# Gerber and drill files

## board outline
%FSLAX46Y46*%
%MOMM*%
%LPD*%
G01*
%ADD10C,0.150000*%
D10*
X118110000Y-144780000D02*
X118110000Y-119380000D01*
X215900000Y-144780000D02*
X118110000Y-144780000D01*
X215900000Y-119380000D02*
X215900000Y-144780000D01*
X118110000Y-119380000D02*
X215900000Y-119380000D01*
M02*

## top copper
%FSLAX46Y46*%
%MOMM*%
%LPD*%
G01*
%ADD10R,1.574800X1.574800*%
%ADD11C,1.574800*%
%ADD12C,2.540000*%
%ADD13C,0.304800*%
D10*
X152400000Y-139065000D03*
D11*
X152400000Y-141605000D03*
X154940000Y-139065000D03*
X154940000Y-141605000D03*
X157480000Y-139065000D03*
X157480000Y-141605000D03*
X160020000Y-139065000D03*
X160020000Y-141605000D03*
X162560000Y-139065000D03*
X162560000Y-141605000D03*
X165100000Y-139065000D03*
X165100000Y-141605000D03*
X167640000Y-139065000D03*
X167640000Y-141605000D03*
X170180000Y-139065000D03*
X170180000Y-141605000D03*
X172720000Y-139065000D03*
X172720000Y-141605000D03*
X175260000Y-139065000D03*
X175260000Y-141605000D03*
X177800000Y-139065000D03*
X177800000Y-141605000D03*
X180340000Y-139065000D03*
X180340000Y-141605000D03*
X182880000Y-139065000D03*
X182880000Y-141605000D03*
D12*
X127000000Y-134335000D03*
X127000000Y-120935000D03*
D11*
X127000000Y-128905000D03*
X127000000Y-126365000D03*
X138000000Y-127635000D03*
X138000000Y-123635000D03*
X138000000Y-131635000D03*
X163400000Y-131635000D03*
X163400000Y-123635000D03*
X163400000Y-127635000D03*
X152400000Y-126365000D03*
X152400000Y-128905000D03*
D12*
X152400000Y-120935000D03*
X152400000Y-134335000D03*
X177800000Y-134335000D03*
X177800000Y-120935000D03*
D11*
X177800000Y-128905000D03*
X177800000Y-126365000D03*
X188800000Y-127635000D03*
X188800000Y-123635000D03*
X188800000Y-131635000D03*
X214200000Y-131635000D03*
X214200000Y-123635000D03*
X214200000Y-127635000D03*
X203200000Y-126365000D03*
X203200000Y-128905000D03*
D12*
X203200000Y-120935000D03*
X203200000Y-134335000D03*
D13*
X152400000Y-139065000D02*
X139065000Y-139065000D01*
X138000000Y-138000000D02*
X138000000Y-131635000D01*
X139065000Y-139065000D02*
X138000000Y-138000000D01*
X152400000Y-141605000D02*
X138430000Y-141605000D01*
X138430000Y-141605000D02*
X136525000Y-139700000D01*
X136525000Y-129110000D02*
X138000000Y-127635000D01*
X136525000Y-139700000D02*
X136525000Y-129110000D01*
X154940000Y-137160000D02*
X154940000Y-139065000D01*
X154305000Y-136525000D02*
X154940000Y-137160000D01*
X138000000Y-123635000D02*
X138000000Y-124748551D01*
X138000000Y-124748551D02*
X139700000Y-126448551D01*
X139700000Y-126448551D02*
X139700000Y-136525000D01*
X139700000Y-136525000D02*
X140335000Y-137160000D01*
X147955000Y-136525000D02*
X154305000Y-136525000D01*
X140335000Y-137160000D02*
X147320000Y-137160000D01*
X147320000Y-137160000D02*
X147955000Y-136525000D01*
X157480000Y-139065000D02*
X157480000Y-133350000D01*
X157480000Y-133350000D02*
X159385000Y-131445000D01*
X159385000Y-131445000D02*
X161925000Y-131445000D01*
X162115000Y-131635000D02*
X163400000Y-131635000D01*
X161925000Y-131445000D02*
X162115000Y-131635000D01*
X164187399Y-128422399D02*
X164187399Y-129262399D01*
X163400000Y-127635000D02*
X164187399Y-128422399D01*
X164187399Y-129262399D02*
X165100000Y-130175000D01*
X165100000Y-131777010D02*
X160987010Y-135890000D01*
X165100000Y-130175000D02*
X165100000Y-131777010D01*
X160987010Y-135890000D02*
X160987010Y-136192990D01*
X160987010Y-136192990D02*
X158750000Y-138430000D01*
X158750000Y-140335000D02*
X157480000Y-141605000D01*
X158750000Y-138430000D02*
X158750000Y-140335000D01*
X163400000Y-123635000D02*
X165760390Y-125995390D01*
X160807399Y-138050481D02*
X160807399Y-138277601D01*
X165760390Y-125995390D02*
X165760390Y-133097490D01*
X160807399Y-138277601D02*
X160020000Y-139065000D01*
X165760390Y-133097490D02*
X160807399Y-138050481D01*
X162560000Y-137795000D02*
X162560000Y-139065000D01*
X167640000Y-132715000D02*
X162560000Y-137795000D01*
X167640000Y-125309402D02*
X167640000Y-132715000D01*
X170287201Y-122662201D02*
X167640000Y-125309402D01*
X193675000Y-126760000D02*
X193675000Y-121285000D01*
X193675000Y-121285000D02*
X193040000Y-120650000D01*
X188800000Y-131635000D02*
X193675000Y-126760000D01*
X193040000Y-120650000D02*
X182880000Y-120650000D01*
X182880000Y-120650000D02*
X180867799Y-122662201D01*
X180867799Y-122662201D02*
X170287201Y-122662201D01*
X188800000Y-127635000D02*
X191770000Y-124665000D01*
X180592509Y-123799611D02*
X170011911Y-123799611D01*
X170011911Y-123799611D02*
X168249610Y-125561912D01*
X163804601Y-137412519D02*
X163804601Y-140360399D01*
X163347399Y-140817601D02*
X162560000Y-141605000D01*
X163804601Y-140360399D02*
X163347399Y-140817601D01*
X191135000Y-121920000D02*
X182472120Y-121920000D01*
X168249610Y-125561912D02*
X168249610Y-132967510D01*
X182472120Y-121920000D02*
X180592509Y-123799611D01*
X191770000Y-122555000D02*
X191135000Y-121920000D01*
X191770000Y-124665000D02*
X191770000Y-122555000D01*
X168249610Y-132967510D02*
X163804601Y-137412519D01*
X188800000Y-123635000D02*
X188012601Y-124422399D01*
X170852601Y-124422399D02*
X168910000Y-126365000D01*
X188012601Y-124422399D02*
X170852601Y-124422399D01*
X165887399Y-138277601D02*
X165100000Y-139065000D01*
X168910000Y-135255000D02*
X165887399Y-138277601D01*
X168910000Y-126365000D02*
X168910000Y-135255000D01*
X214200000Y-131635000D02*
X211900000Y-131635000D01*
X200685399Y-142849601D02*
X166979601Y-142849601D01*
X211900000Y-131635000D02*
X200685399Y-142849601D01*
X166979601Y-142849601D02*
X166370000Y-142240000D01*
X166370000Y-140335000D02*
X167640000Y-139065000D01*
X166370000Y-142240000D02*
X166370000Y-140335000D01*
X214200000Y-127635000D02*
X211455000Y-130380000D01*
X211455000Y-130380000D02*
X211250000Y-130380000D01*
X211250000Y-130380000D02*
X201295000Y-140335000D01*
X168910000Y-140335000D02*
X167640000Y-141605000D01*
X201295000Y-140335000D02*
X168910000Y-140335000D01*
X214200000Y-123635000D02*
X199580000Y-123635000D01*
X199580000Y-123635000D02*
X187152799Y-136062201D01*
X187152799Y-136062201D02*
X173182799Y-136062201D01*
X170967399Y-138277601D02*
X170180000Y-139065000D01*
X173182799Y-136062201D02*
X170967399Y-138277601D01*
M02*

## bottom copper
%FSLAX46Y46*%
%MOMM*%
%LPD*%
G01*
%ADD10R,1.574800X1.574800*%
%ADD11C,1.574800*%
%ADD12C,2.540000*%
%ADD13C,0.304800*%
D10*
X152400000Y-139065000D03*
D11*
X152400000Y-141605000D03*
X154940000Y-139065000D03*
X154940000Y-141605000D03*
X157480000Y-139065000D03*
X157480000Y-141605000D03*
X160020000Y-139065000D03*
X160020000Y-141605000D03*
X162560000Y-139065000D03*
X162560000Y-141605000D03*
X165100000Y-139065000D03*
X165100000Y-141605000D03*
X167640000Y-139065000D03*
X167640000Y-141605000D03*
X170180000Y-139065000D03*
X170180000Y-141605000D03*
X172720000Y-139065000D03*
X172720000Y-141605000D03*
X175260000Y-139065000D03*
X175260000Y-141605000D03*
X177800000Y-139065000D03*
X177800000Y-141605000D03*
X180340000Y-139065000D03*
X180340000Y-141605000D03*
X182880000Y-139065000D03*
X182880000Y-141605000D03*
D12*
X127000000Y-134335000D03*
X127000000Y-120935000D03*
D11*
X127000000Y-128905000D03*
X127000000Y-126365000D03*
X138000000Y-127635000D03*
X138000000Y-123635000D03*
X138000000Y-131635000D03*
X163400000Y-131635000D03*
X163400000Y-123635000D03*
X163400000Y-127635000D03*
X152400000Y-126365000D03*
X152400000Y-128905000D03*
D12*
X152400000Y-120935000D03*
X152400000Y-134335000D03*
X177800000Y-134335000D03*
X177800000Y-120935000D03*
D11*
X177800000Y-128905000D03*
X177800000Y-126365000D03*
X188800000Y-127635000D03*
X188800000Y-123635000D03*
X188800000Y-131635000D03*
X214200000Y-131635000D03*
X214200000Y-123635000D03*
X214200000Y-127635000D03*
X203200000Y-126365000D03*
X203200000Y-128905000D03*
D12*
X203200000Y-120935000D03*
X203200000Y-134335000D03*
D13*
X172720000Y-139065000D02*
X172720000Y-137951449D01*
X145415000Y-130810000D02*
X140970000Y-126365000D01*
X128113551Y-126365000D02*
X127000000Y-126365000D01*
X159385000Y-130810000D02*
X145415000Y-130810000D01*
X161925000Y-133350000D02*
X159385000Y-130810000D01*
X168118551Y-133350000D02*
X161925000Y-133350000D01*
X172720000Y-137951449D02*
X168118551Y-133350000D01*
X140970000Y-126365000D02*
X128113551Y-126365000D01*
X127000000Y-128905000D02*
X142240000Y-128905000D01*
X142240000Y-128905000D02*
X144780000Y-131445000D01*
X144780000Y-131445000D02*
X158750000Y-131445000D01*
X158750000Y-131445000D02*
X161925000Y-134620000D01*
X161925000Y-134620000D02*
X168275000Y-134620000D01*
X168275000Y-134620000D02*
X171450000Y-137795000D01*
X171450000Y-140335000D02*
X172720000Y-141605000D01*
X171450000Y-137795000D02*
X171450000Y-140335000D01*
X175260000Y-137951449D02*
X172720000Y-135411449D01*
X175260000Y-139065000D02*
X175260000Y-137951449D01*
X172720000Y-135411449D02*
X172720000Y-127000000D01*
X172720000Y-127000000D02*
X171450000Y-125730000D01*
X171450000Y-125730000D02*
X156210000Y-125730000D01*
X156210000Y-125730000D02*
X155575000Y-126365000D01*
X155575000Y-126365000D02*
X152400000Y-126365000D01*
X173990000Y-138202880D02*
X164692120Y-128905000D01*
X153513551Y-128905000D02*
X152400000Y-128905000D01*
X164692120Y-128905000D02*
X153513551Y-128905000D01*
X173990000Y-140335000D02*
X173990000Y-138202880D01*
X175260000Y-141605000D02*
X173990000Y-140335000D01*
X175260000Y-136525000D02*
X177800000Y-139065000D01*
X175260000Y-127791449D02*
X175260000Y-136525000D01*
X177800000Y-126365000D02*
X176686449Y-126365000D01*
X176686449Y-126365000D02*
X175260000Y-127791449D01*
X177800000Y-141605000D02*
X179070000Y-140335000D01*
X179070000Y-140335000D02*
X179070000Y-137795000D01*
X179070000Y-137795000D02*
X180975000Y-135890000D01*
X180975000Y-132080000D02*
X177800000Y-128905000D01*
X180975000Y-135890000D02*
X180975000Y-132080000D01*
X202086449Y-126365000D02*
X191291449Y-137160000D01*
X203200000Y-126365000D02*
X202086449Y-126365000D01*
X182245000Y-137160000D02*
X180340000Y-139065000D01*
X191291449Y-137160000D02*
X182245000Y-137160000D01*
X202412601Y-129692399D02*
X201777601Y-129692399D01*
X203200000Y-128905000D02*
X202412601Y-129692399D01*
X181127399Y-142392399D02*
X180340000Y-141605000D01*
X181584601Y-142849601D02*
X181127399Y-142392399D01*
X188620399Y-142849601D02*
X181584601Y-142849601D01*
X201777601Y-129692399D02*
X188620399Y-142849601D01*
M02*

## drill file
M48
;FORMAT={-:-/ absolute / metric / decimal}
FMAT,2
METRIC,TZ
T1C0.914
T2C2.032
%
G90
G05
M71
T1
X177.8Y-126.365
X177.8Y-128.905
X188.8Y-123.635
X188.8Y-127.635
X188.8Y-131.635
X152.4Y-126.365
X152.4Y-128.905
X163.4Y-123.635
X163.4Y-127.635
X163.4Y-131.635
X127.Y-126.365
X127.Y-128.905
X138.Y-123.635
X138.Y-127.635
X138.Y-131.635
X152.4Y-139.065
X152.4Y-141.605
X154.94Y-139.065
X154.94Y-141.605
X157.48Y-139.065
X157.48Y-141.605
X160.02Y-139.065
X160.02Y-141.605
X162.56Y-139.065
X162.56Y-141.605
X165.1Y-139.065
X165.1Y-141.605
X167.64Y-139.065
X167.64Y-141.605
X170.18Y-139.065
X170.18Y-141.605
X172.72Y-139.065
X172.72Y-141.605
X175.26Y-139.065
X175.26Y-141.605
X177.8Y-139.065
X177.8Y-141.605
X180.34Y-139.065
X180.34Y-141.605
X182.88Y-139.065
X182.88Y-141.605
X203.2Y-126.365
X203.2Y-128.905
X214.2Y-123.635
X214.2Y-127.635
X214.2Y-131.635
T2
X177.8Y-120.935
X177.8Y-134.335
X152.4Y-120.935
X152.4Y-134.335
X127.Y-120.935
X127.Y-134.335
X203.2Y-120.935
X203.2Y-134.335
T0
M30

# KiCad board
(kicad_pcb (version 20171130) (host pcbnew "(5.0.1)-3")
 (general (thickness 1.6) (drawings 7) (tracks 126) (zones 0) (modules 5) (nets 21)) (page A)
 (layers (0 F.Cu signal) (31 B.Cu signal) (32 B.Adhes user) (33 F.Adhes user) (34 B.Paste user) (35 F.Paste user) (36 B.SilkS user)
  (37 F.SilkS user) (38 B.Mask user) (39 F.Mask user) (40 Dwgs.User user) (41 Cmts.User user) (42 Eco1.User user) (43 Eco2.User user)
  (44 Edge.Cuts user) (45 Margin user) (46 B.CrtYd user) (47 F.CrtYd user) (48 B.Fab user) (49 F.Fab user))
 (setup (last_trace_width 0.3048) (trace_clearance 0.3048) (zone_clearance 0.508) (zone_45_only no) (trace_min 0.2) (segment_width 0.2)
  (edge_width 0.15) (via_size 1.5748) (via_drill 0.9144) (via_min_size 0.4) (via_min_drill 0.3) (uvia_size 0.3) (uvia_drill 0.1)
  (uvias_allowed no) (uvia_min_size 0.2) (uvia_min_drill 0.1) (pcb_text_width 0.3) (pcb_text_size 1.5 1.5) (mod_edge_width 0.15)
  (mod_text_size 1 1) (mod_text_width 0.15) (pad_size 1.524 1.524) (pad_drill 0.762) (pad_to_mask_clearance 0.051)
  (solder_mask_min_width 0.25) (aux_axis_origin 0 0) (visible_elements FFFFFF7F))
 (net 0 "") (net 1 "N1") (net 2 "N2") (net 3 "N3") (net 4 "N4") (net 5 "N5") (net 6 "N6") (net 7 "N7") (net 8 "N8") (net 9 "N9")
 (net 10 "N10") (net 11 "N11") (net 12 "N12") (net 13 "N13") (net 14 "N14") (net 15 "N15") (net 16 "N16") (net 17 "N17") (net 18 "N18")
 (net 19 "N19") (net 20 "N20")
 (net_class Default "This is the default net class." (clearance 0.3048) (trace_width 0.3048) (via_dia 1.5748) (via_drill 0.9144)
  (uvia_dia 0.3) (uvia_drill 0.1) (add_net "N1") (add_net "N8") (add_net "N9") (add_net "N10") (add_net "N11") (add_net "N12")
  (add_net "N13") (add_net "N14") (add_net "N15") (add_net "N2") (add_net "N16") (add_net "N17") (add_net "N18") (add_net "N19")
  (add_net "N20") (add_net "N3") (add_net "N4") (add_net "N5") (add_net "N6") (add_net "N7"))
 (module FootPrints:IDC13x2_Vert (layer B.Cu) (at 166.37 140.335)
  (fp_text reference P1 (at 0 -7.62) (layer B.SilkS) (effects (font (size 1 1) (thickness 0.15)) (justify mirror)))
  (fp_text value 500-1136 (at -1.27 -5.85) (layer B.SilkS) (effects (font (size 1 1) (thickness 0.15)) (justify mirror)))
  (pad 1 thru_hole rect (at -13.97 -1.27) (size 1.5748 1.5748) (drill 0.9144) (layers *.Cu *.Mask) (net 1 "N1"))
  (pad 2 thru_hole circle (at -13.97 1.27) (size 1.5748 1.5748) (drill 0.9144) (layers *.Cu *.Mask) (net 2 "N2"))
  (pad 3 thru_hole circle (at -11.43 -1.27) (size 1.5748 1.5748) (drill 0.9144) (layers *.Cu *.Mask) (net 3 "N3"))
  (pad 4 thru_hole circle (at -11.43 1.27) (size 1.5748 1.5748) (drill 0.9144) (layers *.Cu *.Mask))
  (pad 5 thru_hole circle (at -8.89 -1.27) (size 1.5748 1.5748) (drill 0.9144) (layers *.Cu *.Mask) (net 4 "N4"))
  (pad 6 thru_hole circle (at -8.89 1.27) (size 1.5748 1.5748) (drill 0.9144) (layers *.Cu *.Mask) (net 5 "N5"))
  (pad 7 thru_hole circle (at -6.35 -1.27) (size 1.5748 1.5748) (drill 0.9144) (layers *.Cu *.Mask) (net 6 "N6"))
  (pad 8 thru_hole circle (at -6.35 1.27) (size 1.5748 1.5748) (drill 0.9144) (layers *.Cu *.Mask))
  (pad 9 thru_hole circle (at -3.81 -1.27) (size 1.5748 1.5748) (drill 0.9144) (layers *.Cu *.Mask) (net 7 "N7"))
  (pad 10 thru_hole circle (at -3.81 1.27) (size 1.5748 1.5748) (drill 0.9144) (layers *.Cu *.Mask) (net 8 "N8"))
  (pad 11 thru_hole circle (at -1.27 -1.27) (size 1.5748 1.5748) (drill 0.9144) (layers *.Cu *.Mask) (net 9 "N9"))
  (pad 12 thru_hole circle (at -1.27 1.27) (size 1.5748 1.5748) (drill 0.9144) (layers *.Cu *.Mask))
  (pad 13 thru_hole circle (at 1.27 -1.27) (size 1.5748 1.5748) (drill 0.9144) (layers *.Cu *.Mask) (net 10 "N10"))
  (pad 14 thru_hole circle (at 1.27 1.27) (size 1.5748 1.5748) (drill 0.9144) (layers *.Cu *.Mask) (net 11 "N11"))
  (pad 15 thru_hole circle (at 3.81 -1.27) (size 1.5748 1.5748) (drill 0.9144) (layers *.Cu *.Mask) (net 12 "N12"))
  (pad 16 thru_hole circle (at 3.81 1.27) (size 1.5748 1.5748) (drill 0.9144) (layers *.Cu *.Mask))
  (pad 17 thru_hole circle (at 6.35 -1.27) (size 1.5748 1.5748) (drill 0.9144) (layers *.Cu *.Mask) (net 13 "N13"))
  (pad 18 thru_hole circle (at 6.35 1.27) (size 1.5748 1.5748) (drill 0.9144) (layers *.Cu *.Mask) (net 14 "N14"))
  (pad 19 thru_hole circle (at 8.89 -1.27) (size 1.5748 1.5748) (drill 0.9144) (layers *.Cu *.Mask) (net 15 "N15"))
  (pad 20 thru_hole circle (at 8.89 1.27) (size 1.5748 1.5748) (drill 0.9144) (layers *.Cu *.Mask) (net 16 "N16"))
  (pad 21 thru_hole circle (at 11.43 -1.27) (size 1.5748 1.5748) (drill 0.9144) (layers *.Cu *.Mask) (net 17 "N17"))
  (pad 22 thru_hole circle (at 11.43 1.27) (size 1.5748 1.5748) (drill 0.9144) (layers *.Cu *.Mask) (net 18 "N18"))
  (pad 23 thru_hole circle (at 13.97 -1.27) (size 1.5748 1.5748) (drill 0.9144) (layers *.Cu *.Mask) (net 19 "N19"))
  (pad 24 thru_hole circle (at 13.97 1.27) (size 1.5748 1.5748) (drill 0.9144) (layers *.Cu *.Mask) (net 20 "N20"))
  (pad 25 thru_hole circle (at 16.51 -1.27) (size 1.5748 1.5748) (drill 0.9144) (layers *.Cu *.Mask))
  (pad 26 thru_hole circle (at 16.51 1.27) (size 1.5748 1.5748) (drill 0.9144) (layers *.Cu *.Mask)))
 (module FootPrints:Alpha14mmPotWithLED (layer F.Cu) (at 127 127.635 90)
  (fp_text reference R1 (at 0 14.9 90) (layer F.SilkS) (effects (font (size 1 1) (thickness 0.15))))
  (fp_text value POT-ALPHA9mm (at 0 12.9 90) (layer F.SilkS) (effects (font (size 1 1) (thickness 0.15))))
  (pad "" thru_hole circle (at -6.7 0 90) (size 2.54 2.54) (drill 2.032) (layers *.Cu *.Mask F.SilkS))
  (pad "" thru_hole circle (at 6.7 0 90) (size 2.54 2.54) (drill 2.032) (layers *.Cu *.Mask F.SilkS))
  (pad 4 thru_hole circle (at -1.27 0 90) (size 1.5748 1.5748) (drill 0.9144) (layers *.Cu *.Mask F.SilkS) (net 14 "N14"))
  (pad 5 thru_hole circle (at 1.27 0 90) (size 1.5748 1.5748) (drill 0.9144) (layers *.Cu *.Mask F.SilkS) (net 13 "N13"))
  (pad 2 thru_hole circle (at 0 11 90) (size 1.5748 1.5748) (drill 0.9144) (layers *.Cu *.Mask F.SilkS) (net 2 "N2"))
  (pad 3 thru_hole circle (at 4 11 90) (size 1.5748 1.5748) (drill 0.9144) (layers *.Cu *.Mask F.SilkS) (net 3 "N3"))
  (pad 1 thru_hole circle (at -4 11 90) (size 1.5748 1.5748) (drill 0.9144) (layers *.Cu *.Mask F.SilkS) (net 1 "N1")))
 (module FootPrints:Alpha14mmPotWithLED (layer F.Cu) (at 152.4 127.635 90)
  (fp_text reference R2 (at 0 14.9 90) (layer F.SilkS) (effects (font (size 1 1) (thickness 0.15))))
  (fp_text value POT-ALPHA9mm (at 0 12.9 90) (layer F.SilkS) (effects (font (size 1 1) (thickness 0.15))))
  (pad 1 thru_hole circle (at -4 11 90) (size 1.5748 1.5748) (drill 0.9144) (layers *.Cu *.Mask F.SilkS) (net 4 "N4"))
  (pad 3 thru_hole circle (at 4 11 90) (size 1.5748 1.5748) (drill 0.9144) (layers *.Cu *.Mask F.SilkS) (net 6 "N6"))
  (pad 2 thru_hole circle (at 0 11 90) (size 1.5748 1.5748) (drill 0.9144) (layers *.Cu *.Mask F.SilkS) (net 5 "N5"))
  (pad 5 thru_hole circle (at 1.27 0 90) (size 1.5748 1.5748) (drill 0.9144) (layers *.Cu *.Mask F.SilkS) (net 15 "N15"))
  (pad 4 thru_hole circle (at -1.27 0 90) (size 1.5748 1.5748) (drill 0.9144) (layers *.Cu *.Mask F.SilkS) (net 16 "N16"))
  (pad "" thru_hole circle (at 6.7 0 90) (size 2.54 2.54) (drill 2.032) (layers *.Cu *.Mask F.SilkS))
  (pad "" thru_hole circle (at -6.7 0 90) (size 2.54 2.54) (drill 2.032) (layers *.Cu *.Mask F.SilkS)))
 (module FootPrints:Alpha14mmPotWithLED (layer F.Cu) (at 177.8 127.635 90)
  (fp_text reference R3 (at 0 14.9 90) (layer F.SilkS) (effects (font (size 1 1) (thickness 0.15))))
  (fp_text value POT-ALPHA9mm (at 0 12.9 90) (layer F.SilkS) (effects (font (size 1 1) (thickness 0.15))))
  (pad "" thru_hole circle (at -6.7 0 90) (size 2.54 2.54) (drill 2.032) (layers *.Cu *.Mask F.SilkS))
  (pad "" thru_hole circle (at 6.7 0 90) (size 2.54 2.54) (drill 2.032) (layers *.Cu *.Mask F.SilkS))
  (pad 4 thru_hole circle (at -1.27 0 90) (size 1.5748 1.5748) (drill 0.9144) (layers *.Cu *.Mask F.SilkS) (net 18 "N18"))
  (pad 5 thru_hole circle (at 1.27 0 90) (size 1.5748 1.5748) (drill 0.9144) (layers *.Cu *.Mask F.SilkS) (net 17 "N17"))
  (pad 2 thru_hole circle (at 0 11 90) (size 1.5748 1.5748) (drill 0.9144) (layers *.Cu *.Mask F.SilkS) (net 8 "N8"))
  (pad 3 thru_hole circle (at 4 11 90) (size 1.5748 1.5748) (drill 0.9144) (layers *.Cu *.Mask F.SilkS) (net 9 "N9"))
  (pad 1 thru_hole circle (at -4 11 90) (size 1.5748 1.5748) (drill 0.9144) (layers *.Cu *.Mask F.SilkS) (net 7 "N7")))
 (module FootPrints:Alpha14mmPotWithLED (layer F.Cu) (at 203.2 127.635 90)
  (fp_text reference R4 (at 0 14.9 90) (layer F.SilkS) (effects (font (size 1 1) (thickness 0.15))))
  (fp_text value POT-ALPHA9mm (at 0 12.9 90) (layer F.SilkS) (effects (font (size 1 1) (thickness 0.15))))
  (pad 1 thru_hole circle (at -4 11 90) (size 1.5748 1.5748) (drill 0.9144) (layers *.Cu *.Mask F.SilkS) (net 10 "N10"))
  (pad 3 thru_hole circle (at 4 11 90) (size 1.5748 1.5748) (drill 0.9144) (layers *.Cu *.Mask F.SilkS) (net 12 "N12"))
  (pad 2 thru_hole circle (at 0 11 90) (size 1.5748 1.5748) (drill 0.9144) (layers *.Cu *.Mask F.SilkS) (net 11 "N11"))
  (pad 5 thru_hole circle (at 1.27 0 90) (size 1.5748 1.5748) (drill 0.9144) (layers *.Cu *.Mask F.SilkS) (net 19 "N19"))
  (pad 4 thru_hole circle (at -1.27 0 90) (size 1.5748 1.5748) (drill 0.9144) (layers *.Cu *.Mask F.SilkS) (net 20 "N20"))
  (pad "" thru_hole circle (at 6.7 0 90) (size 2.54 2.54) (drill 2.032) (layers *.Cu *.Mask F.SilkS))
  (pad "" thru_hole circle (at -6.7 0 90) (size 2.54 2.54) (drill 2.032) (layers *.Cu *.Mask F.SilkS)))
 (gr_line (start 118.11 144.78) (end 118.11 119.38) (layer Edge.Cuts) (width 0.15))
 (gr_line (start 215.9 144.78) (end 118.11 144.78) (layer Edge.Cuts) (width 0.15))
 (gr_line (start 215.9 119.38) (end 215.9 144.78) (layer Edge.Cuts) (width 0.15))
 (gr_line (start 118.11 119.38) (end 215.9 119.38) (layer Edge.Cuts) (width 0.15))
 (segment (start 152.4 139.065) (end 139.065 139.065) (width 0.3048) (layer F.Cu) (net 1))
 (segment (start 138 138) (end 138 131.635) (width 0.3048) (layer F.Cu) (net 1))
 (segment (start 139.065 139.065) (end 138 138) (width 0.3048) (layer F.Cu) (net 1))
 (segment (start 152.4 141.605) (end 138.43 141.605) (width 0.3048) (layer F.Cu) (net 2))
 (segment (start 138.43 141.605) (end 136.525 139.7) (width 0.3048) (layer F.Cu) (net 2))
 (segment (start 136.525 129.11) (end 138 127.635) (width 0.3048) (layer F.Cu) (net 2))
 (segment (start 136.525 139.7) (end 136.525 129.11) (width 0.3048) (layer F.Cu) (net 2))
 (segment (start 154.94 137.16) (end 154.94 139.065) (width 0.3048) (layer F.Cu) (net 3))
 (segment (start 154.305 136.525) (end 154.94 137.16) (width 0.3048) (layer F.Cu) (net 3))
 (segment (start 138 123.635) (end 138 124.748551) (width 0.3048) (layer F.Cu) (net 3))
 (segment (start 138 124.748551) (end 139.7 126.448551) (width 0.3048) (layer F.Cu) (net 3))
 (segment (start 139.7 126.448551) (end 139.7 136.525) (width 0.3048) (layer F.Cu) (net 3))
 (segment (start 139.7 136.525) (end 140.335 137.16) (width 0.3048) (layer F.Cu) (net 3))
 (segment (start 147.955 136.525) (end 154.305 136.525) (width 0.3048) (layer F.Cu) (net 3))
 (segment (start 140.335 137.16) (end 147.32 137.16) (width 0.3048) (layer F.Cu) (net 3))
 (segment (start 147.32 137.16) (end 147.955 136.525) (width 0.3048) (layer F.Cu) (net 3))
 (segment (start 157.48 139.065) (end 157.48 133.35) (width 0.3048) (layer F.Cu) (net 4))
 (segment (start 157.48 133.35) (end 159.385 131.445) (width 0.3048) (layer F.Cu) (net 4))
 (segment (start 159.385 131.445) (end 161.925 131.445) (width 0.3048) (layer F.Cu) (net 4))
 (segment (start 162.115 131.635) (end 163.4 131.635) (width 0.3048) (layer F.Cu) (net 4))
 (segment (start 161.925 131.445) (end 162.115 131.635) (width 0.3048) (layer F.Cu) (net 4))
 (segment (start 164.187399 128.422399) (end 164.187399 129.262399) (width 0.3048) (layer F.Cu) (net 5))
 (segment (start 163.4 127.635) (end 164.187399 128.422399) (width 0.3048) (layer F.Cu) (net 5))
 (segment (start 164.187399 129.262399) (end 165.1 130.175) (width 0.3048) (layer F.Cu) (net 5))
 (segment (start 165.1 131.77701) (end 160.98701 135.89) (width 0.3048) (layer F.Cu) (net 5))
 (segment (start 165.1 130.175) (end 165.1 131.77701) (width 0.3048) (layer F.Cu) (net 5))
 (segment (start 160.98701 135.89) (end 160.98701 136.19299) (width 0.3048) (layer F.Cu) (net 5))
 (segment (start 160.98701 136.19299) (end 158.75 138.43) (width 0.3048) (layer F.Cu) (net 5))
 (segment (start 158.75 140.335) (end 157.48 141.605) (width 0.3048) (layer F.Cu) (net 5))
 (segment (start 158.75 138.43) (end 158.75 140.335) (width 0.3048) (layer F.Cu) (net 5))
 (segment (start 163.4 123.635) (end 165.76039 125.99539) (width 0.3048) (layer F.Cu) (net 6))
 (segment (start 160.807399 138.050481) (end 160.807399 138.277601) (width 0.3048) (layer F.Cu) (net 6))
 (segment (start 165.76039 125.99539) (end 165.76039 133.09749) (width 0.3048) (layer F.Cu) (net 6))
 (segment (start 160.807399 138.277601) (end 160.02 139.065) (width 0.3048) (layer F.Cu) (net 6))
 (segment (start 165.76039 133.09749) (end 160.807399 138.050481) (width 0.3048) (layer F.Cu) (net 6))
 (segment (start 162.56 137.795) (end 162.56 139.065) (width 0.3048) (layer F.Cu) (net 7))
 (segment (start 167.64 132.715) (end 162.56 137.795) (width 0.3048) (layer F.Cu) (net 7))
 (segment (start 167.64 125.309402) (end 167.64 132.715) (width 0.3048) (layer F.Cu) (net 7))
 (segment (start 170.287201 122.662201) (end 167.64 125.309402) (width 0.3048) (layer F.Cu) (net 7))
 (segment (start 193.675 126.76) (end 193.675 121.285) (width 0.3048) (layer F.Cu) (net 7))
 (segment (start 193.675 121.285) (end 193.04 120.65) (width 0.3048) (layer F.Cu) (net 7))
 (segment (start 188.8 131.635) (end 193.675 126.76) (width 0.3048) (layer F.Cu) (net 7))
 (segment (start 193.04 120.65) (end 182.88 120.65) (width 0.3048) (layer F.Cu) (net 7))
 (segment (start 182.88 120.65) (end 180.867799 122.662201) (width 0.3048) (layer F.Cu) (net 7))
 (segment (start 180.867799 122.662201) (end 170.287201 122.662201) (width 0.3048) (layer F.Cu) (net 7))
 (segment (start 188.8 127.635) (end 191.77 124.665) (width 0.3048) (layer F.Cu) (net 8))
 (segment (start 180.592509 123.799611) (end 170.011911 123.799611) (width 0.3048) (layer F.Cu) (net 8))
 (segment (start 170.011911 123.799611) (end 168.24961 125.561912) (width 0.3048) (layer F.Cu) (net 8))
 (segment (start 163.804601 137.412519) (end 163.804601 140.360399) (width 0.3048) (layer F.Cu) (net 8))
 (segment (start 163.347399 140.817601) (end 162.56 141.605) (width 0.3048) (layer F.Cu) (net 8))
 (segment (start 163.804601 140.360399) (end 163.347399 140.817601) (width 0.3048) (layer F.Cu) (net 8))
 (segment (start 191.135 121.92) (end 182.47212 121.92) (width 0.3048) (layer F.Cu) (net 8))
 (segment (start 168.24961 125.561912) (end 168.24961 132.96751) (width 0.3048) (layer F.Cu) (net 8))
 (segment (start 182.47212 121.92) (end 180.592509 123.799611) (width 0.3048) (layer F.Cu) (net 8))
 (segment (start 191.77 122.555) (end 191.135 121.92) (width 0.3048) (layer F.Cu) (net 8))
 (segment (start 191.77 124.665) (end 191.77 122.555) (width 0.3048) (layer F.Cu) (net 8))
 (segment (start 168.24961 132.96751) (end 163.804601 137.412519) (width 0.3048) (layer F.Cu) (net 8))
 (segment (start 188.8 123.635) (end 188.012601 124.422399) (width 0.3048) (layer F.Cu) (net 9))
 (segment (start 170.852601 124.422399) (end 168.91 126.365) (width 0.3048) (layer F.Cu) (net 9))
 (segment (start 188.012601 124.422399) (end 170.852601 124.422399) (width 0.3048) (layer F.Cu) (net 9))
 (segment (start 165.887399 138.277601) (end 165.1 139.065) (width 0.3048) (layer F.Cu) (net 9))
 (segment (start 168.91 135.255) (end 165.887399 138.277601) (width 0.3048) (layer F.Cu) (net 9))
 (segment (start 168.91 126.365) (end 168.91 135.255) (width 0.3048) (layer F.Cu) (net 9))
 (segment (start 214.2 131.635) (end 211.9 131.635) (width 0.3048) (layer F.Cu) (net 10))
 (segment (start 200.685399 142.849601) (end 166.979601 142.849601) (width 0.3048) (layer F.Cu) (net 10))
 (segment (start 211.9 131.635) (end 200.685399 142.849601) (width 0.3048) (layer F.Cu) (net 10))
 (segment (start 166.979601 142.849601) (end 166.37 142.24) (width 0.3048) (layer F.Cu) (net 10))
 (segment (start 166.37 140.335) (end 167.64 139.065) (width 0.3048) (layer F.Cu) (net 10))
 (segment (start 166.37 142.24) (end 166.37 140.335) (width 0.3048) (layer F.Cu) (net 10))
 (segment (start 214.2 127.635) (end 211.455 130.38) (width 0.3048) (layer F.Cu) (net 11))
 (segment (start 211.455 130.38) (end 211.25 130.38) (width 0.3048) (layer F.Cu) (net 11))
 (segment (start 211.25 130.38) (end 201.295 140.335) (width 0.3048) (layer F.Cu) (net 11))
 (segment (start 168.91 140.335) (end 167.64 141.605) (width 0.3048) (layer F.Cu) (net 11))
 (segment (start 201.295 140.335) (end 168.91 140.335) (width 0.3048) (layer F.Cu) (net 11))
 (segment (start 214.2 123.635) (end 199.58 123.635) (width 0.3048) (layer F.Cu) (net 12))
 (segment (start 199.58 123.635) (end 187.152799 136.062201) (width 0.3048) (layer F.Cu) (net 12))
 (segment (start 187.152799 136.062201) (end 173.182799 136.062201) (width 0.3048) (layer F.Cu) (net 12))
 (segment (start 170.967399 138.277601) (end 170.18 139.065) (width 0.3048) (layer F.Cu) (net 12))
 (segment (start 173.182799 136.062201) (end 170.967399 138.277601) (width 0.3048) (layer F.Cu) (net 12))
 (segment (start 172.72 139.065) (end 172.72 137.951449) (width 0.3048) (layer B.Cu) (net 13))
 (segment (start 145.415 130.81) (end 140.97 126.365) (width 0.3048) (layer B.Cu) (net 13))
 (segment (start 128.113551 126.365) (end 127 126.365) (width 0.3048) (layer B.Cu) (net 13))
 (segment (start 159.385 130.81) (end 145.415 130.81) (width 0.3048) (layer B.Cu) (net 13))
 (segment (start 161.925 133.35) (end 159.385 130.81) (width 0.3048) (layer B.Cu) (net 13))
 (segment (start 168.118551 133.35) (end 161.925 133.35) (width 0.3048) (layer B.Cu) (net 13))
 (segment (start 172.72 137.951449) (end 168.118551 133.35) (width 0.3048) (layer B.Cu) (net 13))
 (segment (start 140.97 126.365) (end 128.113551 126.365) (width 0.3048) (layer B.Cu) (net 13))
 (segment (start 127 128.905) (end 142.24 128.905) (width 0.3048) (layer B.Cu) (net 14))
 (segment (start 142.24 128.905) (end 144.78 131.445) (width 0.3048) (layer B.Cu) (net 14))
 (segment (start 144.78 131.445) (end 158.75 131.445) (width 0.3048) (layer B.Cu) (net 14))
 (segment (start 158.75 131.445) (end 161.925 134.62) (width 0.3048) (layer B.Cu) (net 14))
 (segment (start 161.925 134.62) (end 168.275 134.62) (width 0.3048) (layer B.Cu) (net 14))
 (segment (start 168.275 134.62) (end 171.45 137.795) (width 0.3048) (layer B.Cu) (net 14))
 (segment (start 171.45 140.335) (end 172.72 141.605) (width 0.3048) (layer B.Cu) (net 14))
 (segment (start 171.45 137.795) (end 171.45 140.335) (width 0.3048) (layer B.Cu) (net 14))
 (segment (start 175.26 137.951449) (end 172.72 135.411449) (width 0.3048) (layer B.Cu) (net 15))
 (segment (start 175.26 139.065) (end 175.26 137.951449) (width 0.3048) (layer B.Cu) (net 15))
 (segment (start 172.72 135.411449) (end 172.72 127) (width 0.3048) (layer B.Cu) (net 15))
 (segment (start 172.72 127) (end 171.45 125.73) (width 0.3048) (layer B.Cu) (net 15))
 (segment (start 171.45 125.73) (end 156.21 125.73) (width 0.3048) (layer B.Cu) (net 15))
 (segment (start 156.21 125.73) (end 155.575 126.365) (width 0.3048) (layer B.Cu) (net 15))
 (segment (start 155.575 126.365) (end 152.4 126.365) (width 0.3048) (layer B.Cu) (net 15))
 (segment (start 173.99 138.20288) (end 164.69212 128.905) (width 0.3048) (layer B.Cu) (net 16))
 (segment (start 153.513551 128.905) (end 152.4 128.905) (width 0.3048) (layer B.Cu) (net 16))
 (segment (start 164.69212 128.905) (end 153.513551 128.905) (width 0.3048) (layer B.Cu) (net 16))
 (segment (start 173.99 140.335) (end 173.99 138.20288) (width 0.3048) (layer B.Cu) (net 16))
 (segment (start 175.26 141.605) (end 173.99 140.335) (width 0.3048) (layer B.Cu) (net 16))
 (segment (start 175.26 136.525) (end 177.8 139.065) (width 0.3048) (layer B.Cu) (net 17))
 (segment (start 175.26 127.791449) (end 175.26 136.525) (width 0.3048) (layer B.Cu) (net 17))
 (segment (start 177.8 126.365) (end 176.686449 126.365) (width 0.3048) (layer B.Cu) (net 17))
 (segment (start 176.686449 126.365) (end 175.26 127.791449) (width 0.3048) (layer B.Cu) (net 17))
 (segment (start 177.8 141.605) (end 179.07 140.335) (width 0.3048) (layer B.Cu) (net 18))
 (segment (start 179.07 140.335) (end 179.07 137.795) (width 0.3048) (layer B.Cu) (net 18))
 (segment (start 179.07 137.795) (end 180.975 135.89) (width 0.3048) (layer B.Cu) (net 18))
 (segment (start 180.975 132.08) (end 177.8 128.905) (width 0.3048) (layer B.Cu) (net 18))
 (segment (start 180.975 135.89) (end 180.975 132.08) (width 0.3048) (layer B.Cu) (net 18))
 (segment (start 202.086449 126.365) (end 191.291449 137.16) (width 0.3048) (layer B.Cu) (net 19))
 (segment (start 203.2 126.365) (end 202.086449 126.365) (width 0.3048) (layer B.Cu) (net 19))
 (segment (start 182.245 137.16) (end 180.34 139.065) (width 0.3048) (layer B.Cu) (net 19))
 (segment (start 191.291449 137.16) (end 182.245 137.16) (width 0.3048) (layer B.Cu) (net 19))
 (segment (start 202.412601 129.692399) (end 201.777601 129.692399) (width 0.3048) (layer B.Cu) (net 20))
 (segment (start 203.2 128.905) (end 202.412601 129.692399) (width 0.3048) (layer B.Cu) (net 20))
 (segment (start 181.127399 142.392399) (end 180.34 141.605) (width 0.3048) (layer B.Cu) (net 20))
 (segment (start 181.584601 142.849601) (end 181.127399 142.392399) (width 0.3048) (layer B.Cu) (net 20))
 (segment (start 188.620399 142.849601) (end 181.584601 142.849601) (width 0.3048) (layer B.Cu) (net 20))
 (segment (start 201.777601 129.692399) (end 188.620399 142.849601) (width 0.3048) (layer B.Cu) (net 20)))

